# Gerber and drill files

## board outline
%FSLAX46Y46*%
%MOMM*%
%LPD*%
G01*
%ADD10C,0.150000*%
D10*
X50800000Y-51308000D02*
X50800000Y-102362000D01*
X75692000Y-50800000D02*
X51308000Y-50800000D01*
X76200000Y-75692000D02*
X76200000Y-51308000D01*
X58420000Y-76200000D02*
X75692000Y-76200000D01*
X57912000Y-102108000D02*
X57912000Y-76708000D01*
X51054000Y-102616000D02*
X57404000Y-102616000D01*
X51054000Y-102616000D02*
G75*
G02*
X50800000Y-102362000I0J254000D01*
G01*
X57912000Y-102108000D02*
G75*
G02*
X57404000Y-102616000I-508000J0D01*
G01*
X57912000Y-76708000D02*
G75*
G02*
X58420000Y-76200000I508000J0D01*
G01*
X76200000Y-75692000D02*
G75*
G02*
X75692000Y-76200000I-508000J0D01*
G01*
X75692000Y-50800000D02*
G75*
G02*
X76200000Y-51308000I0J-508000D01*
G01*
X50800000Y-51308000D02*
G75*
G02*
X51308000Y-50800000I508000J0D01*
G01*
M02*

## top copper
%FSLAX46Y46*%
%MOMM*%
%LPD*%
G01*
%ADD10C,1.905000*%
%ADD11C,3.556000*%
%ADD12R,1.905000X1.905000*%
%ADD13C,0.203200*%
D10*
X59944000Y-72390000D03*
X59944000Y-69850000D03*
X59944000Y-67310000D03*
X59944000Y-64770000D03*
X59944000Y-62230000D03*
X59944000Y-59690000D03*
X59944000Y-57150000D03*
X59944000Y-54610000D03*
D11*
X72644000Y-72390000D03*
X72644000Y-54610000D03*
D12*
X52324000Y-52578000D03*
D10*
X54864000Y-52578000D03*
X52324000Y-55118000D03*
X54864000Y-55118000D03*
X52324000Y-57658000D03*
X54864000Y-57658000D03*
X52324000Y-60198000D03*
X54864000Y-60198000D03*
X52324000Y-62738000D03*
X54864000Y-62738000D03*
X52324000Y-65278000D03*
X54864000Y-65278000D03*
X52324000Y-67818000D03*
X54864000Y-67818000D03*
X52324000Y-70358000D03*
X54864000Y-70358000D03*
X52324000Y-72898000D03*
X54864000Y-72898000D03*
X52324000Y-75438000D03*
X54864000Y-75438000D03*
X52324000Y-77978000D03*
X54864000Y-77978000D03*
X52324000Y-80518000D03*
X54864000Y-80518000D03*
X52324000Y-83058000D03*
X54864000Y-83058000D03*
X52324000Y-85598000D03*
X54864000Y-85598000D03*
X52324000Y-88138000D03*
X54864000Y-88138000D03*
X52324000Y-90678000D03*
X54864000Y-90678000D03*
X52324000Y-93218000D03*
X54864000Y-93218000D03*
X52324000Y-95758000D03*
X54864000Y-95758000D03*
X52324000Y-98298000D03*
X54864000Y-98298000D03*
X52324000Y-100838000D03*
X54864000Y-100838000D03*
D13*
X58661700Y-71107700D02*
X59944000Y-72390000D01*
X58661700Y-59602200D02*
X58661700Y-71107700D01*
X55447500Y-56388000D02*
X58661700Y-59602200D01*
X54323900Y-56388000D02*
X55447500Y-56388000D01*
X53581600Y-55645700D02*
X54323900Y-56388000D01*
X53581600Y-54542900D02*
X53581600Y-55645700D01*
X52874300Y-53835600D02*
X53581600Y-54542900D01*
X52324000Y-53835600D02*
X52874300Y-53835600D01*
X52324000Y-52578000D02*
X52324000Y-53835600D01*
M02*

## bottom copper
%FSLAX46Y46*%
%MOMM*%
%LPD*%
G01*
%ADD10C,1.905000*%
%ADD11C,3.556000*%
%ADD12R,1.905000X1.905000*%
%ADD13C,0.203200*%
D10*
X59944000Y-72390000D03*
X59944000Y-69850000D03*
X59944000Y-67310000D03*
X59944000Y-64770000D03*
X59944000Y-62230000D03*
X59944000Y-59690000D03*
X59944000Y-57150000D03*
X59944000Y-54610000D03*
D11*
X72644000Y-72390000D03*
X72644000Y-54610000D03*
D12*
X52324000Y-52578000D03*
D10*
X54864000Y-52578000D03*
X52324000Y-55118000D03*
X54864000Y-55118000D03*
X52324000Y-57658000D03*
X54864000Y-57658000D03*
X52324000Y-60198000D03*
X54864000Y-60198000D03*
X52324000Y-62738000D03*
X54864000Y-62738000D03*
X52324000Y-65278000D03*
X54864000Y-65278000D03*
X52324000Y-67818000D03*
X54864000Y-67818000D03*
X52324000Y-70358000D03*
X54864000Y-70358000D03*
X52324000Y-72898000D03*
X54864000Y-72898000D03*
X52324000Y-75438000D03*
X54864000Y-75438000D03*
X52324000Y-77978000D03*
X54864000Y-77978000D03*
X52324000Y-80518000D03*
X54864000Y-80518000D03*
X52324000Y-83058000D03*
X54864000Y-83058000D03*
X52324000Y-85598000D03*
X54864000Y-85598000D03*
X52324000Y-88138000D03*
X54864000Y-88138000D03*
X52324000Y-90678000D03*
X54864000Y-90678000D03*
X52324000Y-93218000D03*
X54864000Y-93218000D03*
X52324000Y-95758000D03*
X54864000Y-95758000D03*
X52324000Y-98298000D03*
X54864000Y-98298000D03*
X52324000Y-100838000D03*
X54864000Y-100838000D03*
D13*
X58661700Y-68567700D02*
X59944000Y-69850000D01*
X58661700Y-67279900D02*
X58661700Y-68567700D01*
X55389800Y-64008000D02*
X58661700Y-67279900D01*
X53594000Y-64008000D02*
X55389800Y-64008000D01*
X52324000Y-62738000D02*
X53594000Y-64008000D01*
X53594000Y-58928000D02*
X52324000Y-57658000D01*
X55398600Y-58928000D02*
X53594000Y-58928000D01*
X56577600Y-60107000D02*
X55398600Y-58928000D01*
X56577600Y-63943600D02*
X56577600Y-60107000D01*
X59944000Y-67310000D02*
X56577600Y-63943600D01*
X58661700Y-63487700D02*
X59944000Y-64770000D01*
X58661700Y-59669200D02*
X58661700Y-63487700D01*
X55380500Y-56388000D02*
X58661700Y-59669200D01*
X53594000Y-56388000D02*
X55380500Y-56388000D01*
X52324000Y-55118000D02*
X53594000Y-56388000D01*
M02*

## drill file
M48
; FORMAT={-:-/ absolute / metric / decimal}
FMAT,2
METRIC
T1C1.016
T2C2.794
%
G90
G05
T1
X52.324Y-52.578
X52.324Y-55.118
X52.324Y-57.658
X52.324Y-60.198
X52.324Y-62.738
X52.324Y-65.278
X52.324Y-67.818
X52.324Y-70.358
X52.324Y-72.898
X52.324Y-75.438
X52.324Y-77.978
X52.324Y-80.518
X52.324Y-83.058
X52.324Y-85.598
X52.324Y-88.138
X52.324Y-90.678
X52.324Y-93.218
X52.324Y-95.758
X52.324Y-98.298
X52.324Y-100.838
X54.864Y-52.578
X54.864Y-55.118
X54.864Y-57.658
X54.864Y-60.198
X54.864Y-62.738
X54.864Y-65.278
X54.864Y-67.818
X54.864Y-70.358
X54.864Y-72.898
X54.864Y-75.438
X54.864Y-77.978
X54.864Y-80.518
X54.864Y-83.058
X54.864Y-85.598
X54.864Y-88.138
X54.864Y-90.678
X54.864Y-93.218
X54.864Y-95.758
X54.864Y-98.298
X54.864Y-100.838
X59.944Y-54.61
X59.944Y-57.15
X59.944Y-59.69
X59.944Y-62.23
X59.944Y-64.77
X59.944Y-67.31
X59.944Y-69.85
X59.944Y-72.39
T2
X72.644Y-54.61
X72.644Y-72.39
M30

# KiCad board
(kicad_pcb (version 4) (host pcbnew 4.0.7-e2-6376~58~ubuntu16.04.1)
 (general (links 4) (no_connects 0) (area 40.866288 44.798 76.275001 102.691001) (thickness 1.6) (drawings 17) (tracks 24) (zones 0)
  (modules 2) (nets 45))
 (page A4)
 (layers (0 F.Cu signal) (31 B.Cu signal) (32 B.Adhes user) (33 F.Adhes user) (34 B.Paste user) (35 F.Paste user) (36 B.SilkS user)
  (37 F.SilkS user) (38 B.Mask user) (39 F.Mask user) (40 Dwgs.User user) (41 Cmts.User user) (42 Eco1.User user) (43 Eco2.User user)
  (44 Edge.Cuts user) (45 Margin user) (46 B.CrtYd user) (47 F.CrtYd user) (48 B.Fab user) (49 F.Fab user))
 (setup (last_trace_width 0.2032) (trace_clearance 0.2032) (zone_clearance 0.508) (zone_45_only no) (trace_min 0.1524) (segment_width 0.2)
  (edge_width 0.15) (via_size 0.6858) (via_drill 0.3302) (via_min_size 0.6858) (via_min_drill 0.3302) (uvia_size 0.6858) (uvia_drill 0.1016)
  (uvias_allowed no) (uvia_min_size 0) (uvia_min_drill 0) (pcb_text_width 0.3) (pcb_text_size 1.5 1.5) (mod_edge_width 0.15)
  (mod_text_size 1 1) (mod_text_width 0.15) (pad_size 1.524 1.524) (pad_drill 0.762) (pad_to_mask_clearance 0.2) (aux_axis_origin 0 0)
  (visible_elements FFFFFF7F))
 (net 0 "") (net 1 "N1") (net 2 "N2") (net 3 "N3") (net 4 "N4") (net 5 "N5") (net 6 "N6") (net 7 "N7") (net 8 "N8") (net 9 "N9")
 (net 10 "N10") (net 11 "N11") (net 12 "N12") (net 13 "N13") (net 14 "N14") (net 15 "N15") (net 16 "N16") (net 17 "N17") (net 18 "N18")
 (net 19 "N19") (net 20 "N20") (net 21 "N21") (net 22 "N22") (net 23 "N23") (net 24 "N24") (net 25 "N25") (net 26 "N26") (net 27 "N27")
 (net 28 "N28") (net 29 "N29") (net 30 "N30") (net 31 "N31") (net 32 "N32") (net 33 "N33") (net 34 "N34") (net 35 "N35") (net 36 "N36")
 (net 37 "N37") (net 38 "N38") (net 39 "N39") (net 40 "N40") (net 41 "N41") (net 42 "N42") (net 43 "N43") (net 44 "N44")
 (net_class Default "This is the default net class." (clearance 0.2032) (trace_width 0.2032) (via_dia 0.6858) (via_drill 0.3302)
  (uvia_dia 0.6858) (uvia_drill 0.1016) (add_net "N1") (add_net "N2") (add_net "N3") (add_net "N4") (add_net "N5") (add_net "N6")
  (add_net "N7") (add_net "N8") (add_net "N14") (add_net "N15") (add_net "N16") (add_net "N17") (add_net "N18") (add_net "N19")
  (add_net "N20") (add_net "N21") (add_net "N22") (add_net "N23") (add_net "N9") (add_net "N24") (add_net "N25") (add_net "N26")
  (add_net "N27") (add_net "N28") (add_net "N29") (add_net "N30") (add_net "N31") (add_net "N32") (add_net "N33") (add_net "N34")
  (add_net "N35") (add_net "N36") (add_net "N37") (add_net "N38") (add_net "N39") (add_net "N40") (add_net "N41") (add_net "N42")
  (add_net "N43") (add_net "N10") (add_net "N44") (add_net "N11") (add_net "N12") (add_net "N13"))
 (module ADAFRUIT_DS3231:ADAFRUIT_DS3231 (layer B.Cu) (at 59.944 63.5)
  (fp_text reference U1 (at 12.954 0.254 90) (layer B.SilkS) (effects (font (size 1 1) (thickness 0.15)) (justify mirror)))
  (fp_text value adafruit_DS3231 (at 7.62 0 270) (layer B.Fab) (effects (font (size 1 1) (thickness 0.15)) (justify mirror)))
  (pad 1 thru_hole circle (at 0 8.89) (size 1.905 1.905) (drill 1.016) (layers *.Cu *.Mask) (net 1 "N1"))
  (pad 2 thru_hole circle (at 0 6.35) (size 1.905 1.905) (drill 1.016) (layers *.Cu *.Mask) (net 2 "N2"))
  (pad 3 thru_hole circle (at 0 3.81) (size 1.905 1.905) (drill 1.016) (layers *.Cu *.Mask) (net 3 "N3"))
  (pad 4 thru_hole circle (at 0 1.27) (size 1.905 1.905) (drill 1.016) (layers *.Cu *.Mask) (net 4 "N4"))
  (pad 5 thru_hole circle (at 0 -1.27) (size 1.905 1.905) (drill 1.016) (layers *.Cu *.Mask) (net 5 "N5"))
  (pad 6 thru_hole circle (at 0 -3.81) (size 1.905 1.905) (drill 1.016) (layers *.Cu *.Mask) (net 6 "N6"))
  (pad 7 thru_hole circle (at 0 -6.35) (size 1.905 1.905) (drill 1.016) (layers *.Cu *.Mask) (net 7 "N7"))
  (pad 8 thru_hole circle (at 0 -8.89) (size 1.905 1.905) (drill 1.016) (layers *.Cu *.Mask) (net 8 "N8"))
  (pad "" thru_hole circle (at 12.7 8.89) (size 3.556 3.556) (drill 2.794) (layers *.Cu *.Mask))
  (pad "" thru_hole circle (at 12.7 -8.89) (size 3.556 3.556) (drill 2.794) (layers *.Cu *.Mask)))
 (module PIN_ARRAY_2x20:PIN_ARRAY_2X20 (layer F.Cu) (at 53.594 76.708)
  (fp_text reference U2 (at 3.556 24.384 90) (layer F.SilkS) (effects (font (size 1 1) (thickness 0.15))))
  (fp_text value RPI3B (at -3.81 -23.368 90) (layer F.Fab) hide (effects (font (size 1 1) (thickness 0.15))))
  (pad 1 thru_hole rect (at -1.27 -24.13) (size 1.905 1.905) (drill 1.016) (layers *.Cu *.Mask) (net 1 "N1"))
  (pad 2 thru_hole circle (at 1.27 -24.13) (size 1.905 1.905) (drill 1.016) (layers *.Cu *.Mask) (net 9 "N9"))
  (pad 3 thru_hole circle (at -1.27 -21.59) (size 1.905 1.905) (drill 1.016) (layers *.Cu *.Mask) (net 4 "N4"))
  (pad 4 thru_hole circle (at 1.27 -21.59) (size 1.905 1.905) (drill 1.016) (layers *.Cu *.Mask) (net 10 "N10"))
  (pad 5 thru_hole circle (at -1.27 -19.05) (size 1.905 1.905) (drill 1.016) (layers *.Cu *.Mask) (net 3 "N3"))
  (pad 6 thru_hole circle (at 1.27 -19.05) (size 1.905 1.905) (drill 1.016) (layers *.Cu *.Mask) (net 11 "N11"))
  (pad 7 thru_hole circle (at -1.27 -16.51) (size 1.905 1.905) (drill 1.016) (layers *.Cu *.Mask) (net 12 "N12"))
  (pad 8 thru_hole circle (at 1.27 -16.51) (size 1.905 1.905) (drill 1.016) (layers *.Cu *.Mask) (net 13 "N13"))
  (pad 9 thru_hole circle (at -1.27 -13.97) (size 1.905 1.905) (drill 1.016) (layers *.Cu *.Mask) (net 2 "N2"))
  (pad 10 thru_hole circle (at 1.27 -13.97) (size 1.905 1.905) (drill 1.016) (layers *.Cu *.Mask) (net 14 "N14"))
  (pad 11 thru_hole circle (at -1.27 -11.43) (size 1.905 1.905) (drill 1.016) (layers *.Cu *.Mask) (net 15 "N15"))
  (pad 12 thru_hole circle (at 1.27 -11.43) (size 1.905 1.905) (drill 1.016) (layers *.Cu *.Mask) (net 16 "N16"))
  (pad 13 thru_hole circle (at -1.27 -8.89) (size 1.905 1.905) (drill 1.016) (layers *.Cu *.Mask) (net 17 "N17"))
  (pad 14 thru_hole circle (at 1.27 -8.89) (size 1.905 1.905) (drill 1.016) (layers *.Cu *.Mask) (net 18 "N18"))
  (pad 15 thru_hole circle (at -1.27 -6.35) (size 1.905 1.905) (drill 1.016) (layers *.Cu *.Mask) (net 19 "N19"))
  (pad 16 thru_hole circle (at 1.27 -6.35) (size 1.905 1.905) (drill 1.016) (layers *.Cu *.Mask) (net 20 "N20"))
  (pad 17 thru_hole circle (at -1.27 -3.81) (size 1.905 1.905) (drill 1.016) (layers *.Cu *.Mask) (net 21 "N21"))
  (pad 18 thru_hole circle (at 1.27 -3.81) (size 1.905 1.905) (drill 1.016) (layers *.Cu *.Mask) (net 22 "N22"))
  (pad 19 thru_hole circle (at -1.27 -1.27) (size 1.905 1.905) (drill 1.016) (layers *.Cu *.Mask) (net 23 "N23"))
  (pad 20 thru_hole circle (at 1.27 -1.27) (size 1.905 1.905) (drill 1.016) (layers *.Cu *.Mask) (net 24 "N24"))
  (pad 21 thru_hole circle (at -1.27 1.27) (size 1.905 1.905) (drill 1.016) (layers *.Cu *.Mask) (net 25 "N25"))
  (pad 22 thru_hole circle (at 1.27 1.27) (size 1.905 1.905) (drill 1.016) (layers *.Cu *.Mask) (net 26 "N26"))
  (pad 23 thru_hole circle (at -1.27 3.81) (size 1.905 1.905) (drill 1.016) (layers *.Cu *.Mask) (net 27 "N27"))
  (pad 24 thru_hole circle (at 1.27 3.81) (size 1.905 1.905) (drill 1.016) (layers *.Cu *.Mask) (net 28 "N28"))
  (pad 25 thru_hole circle (at -1.27 6.35) (size 1.905 1.905) (drill 1.016) (layers *.Cu *.Mask) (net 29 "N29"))
  (pad 26 thru_hole circle (at 1.27 6.35) (size 1.905 1.905) (drill 1.016) (layers *.Cu *.Mask) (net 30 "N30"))
  (pad 27 thru_hole circle (at -1.27 8.89) (size 1.905 1.905) (drill 1.016) (layers *.Cu *.Mask) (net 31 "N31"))
  (pad 28 thru_hole circle (at 1.27 8.89) (size 1.905 1.905) (drill 1.016) (layers *.Cu *.Mask) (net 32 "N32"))
  (pad 29 thru_hole circle (at -1.27 11.43) (size 1.905 1.905) (drill 1.016) (layers *.Cu *.Mask) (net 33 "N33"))
  (pad 30 thru_hole circle (at 1.27 11.43) (size 1.905 1.905) (drill 1.016) (layers *.Cu *.Mask) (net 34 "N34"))
  (pad 31 thru_hole circle (at -1.27 13.97) (size 1.905 1.905) (drill 1.016) (layers *.Cu *.Mask) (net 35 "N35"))
  (pad 32 thru_hole circle (at 1.27 13.97) (size 1.905 1.905) (drill 1.016) (layers *.Cu *.Mask) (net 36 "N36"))
  (pad 33 thru_hole circle (at -1.27 16.51) (size 1.905 1.905) (drill 1.016) (layers *.Cu *.Mask) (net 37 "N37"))
  (pad 34 thru_hole circle (at 1.27 16.51) (size 1.905 1.905) (drill 1.016) (layers *.Cu *.Mask) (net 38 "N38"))
  (pad 35 thru_hole circle (at -1.27 19.05) (size 1.905 1.905) (drill 1.016) (layers *.Cu *.Mask) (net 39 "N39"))
  (pad 36 thru_hole circle (at 1.27 19.05) (size 1.905 1.905) (drill 1.016) (layers *.Cu *.Mask) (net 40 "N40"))
  (pad 37 thru_hole circle (at -1.27 21.59) (size 1.905 1.905) (drill 1.016) (layers *.Cu *.Mask) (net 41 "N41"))
  (pad 38 thru_hole circle (at 1.27 21.59) (size 1.905 1.905) (drill 1.016) (layers *.Cu *.Mask) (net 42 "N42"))
  (pad 39 thru_hole circle (at -1.27 24.13) (size 1.905 1.905) (drill 1.016) (layers *.Cu *.Mask) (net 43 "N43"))
  (pad 40 thru_hole circle (at 1.27 24.13) (size 1.905 1.905) (drill 1.016) (layers *.Cu *.Mask) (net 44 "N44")))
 (gr_line (start 50.8 51.308) (end 50.8 102.362) (angle 90) (layer Edge.Cuts) (width 0.15))
 (gr_line (start 75.692 50.8) (end 51.308 50.8) (angle 90) (layer Edge.Cuts) (width 0.15))
 (gr_line (start 76.2 75.692) (end 76.2 51.308) (angle 90) (layer Edge.Cuts) (width 0.15))
 (gr_line (start 58.42 76.2) (end 75.692 76.2) (angle 90) (layer Edge.Cuts) (width 0.15))
 (gr_line (start 57.912 102.108) (end 57.912 76.708) (angle 90) (layer Edge.Cuts) (width 0.15))
 (gr_line (start 51.054 102.616) (end 57.404 102.616) (angle 90) (layer Edge.Cuts) (width 0.15))
 (gr_arc (start 51.054 102.362) (end 51.054 102.616) (angle 90) (layer Edge.Cuts) (width 0.15))
 (gr_arc (start 57.404 102.108) (end 57.912 102.108) (angle 90) (layer Edge.Cuts) (width 0.15))
 (gr_arc (start 58.42 76.708) (end 57.912 76.708) (angle 90) (layer Edge.Cuts) (width 0.15))
 (gr_arc (start 75.692 75.692) (end 76.2 75.692) (angle 90) (layer Edge.Cuts) (width 0.15))
 (gr_arc (start 75.692 51.308) (end 75.692 50.8) (angle 90) (layer Edge.Cuts) (width 0.15))
 (gr_arc (start 51.308 51.308) (end 50.8 51.308) (angle 90) (layer Edge.Cuts) (width 0.15))
 (segment (start 58.6617 71.1077) (end 59.944 72.39) (width 0.2032) (layer F.Cu) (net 1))
 (segment (start 58.6617 59.6022) (end 58.6617 71.1077) (width 0.2032) (layer F.Cu) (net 1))
 (segment (start 55.4475 56.388) (end 58.6617 59.6022) (width 0.2032) (layer F.Cu) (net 1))
 (segment (start 54.3239 56.388) (end 55.4475 56.388) (width 0.2032) (layer F.Cu) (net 1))
 (segment (start 53.5816 55.6457) (end 54.3239 56.388) (width 0.2032) (layer F.Cu) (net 1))
 (segment (start 53.5816 54.5429) (end 53.5816 55.6457) (width 0.2032) (layer F.Cu) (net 1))
 (segment (start 52.8743 53.8356) (end 53.5816 54.5429) (width 0.2032) (layer F.Cu) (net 1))
 (segment (start 52.324 53.8356) (end 52.8743 53.8356) (width 0.2032) (layer F.Cu) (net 1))
 (segment (start 52.324 52.578) (end 52.324 53.8356) (width 0.2032) (layer F.Cu) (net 1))
 (segment (start 58.6617 68.5677) (end 59.944 69.85) (width 0.2032) (layer B.Cu) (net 2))
 (segment (start 58.6617 67.2799) (end 58.6617 68.5677) (width 0.2032) (layer B.Cu) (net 2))
 (segment (start 55.3898 64.008) (end 58.6617 67.2799) (width 0.2032) (layer B.Cu) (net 2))
 (segment (start 53.594 64.008) (end 55.3898 64.008) (width 0.2032) (layer B.Cu) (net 2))
 (segment (start 52.324 62.738) (end 53.594 64.008) (width 0.2032) (layer B.Cu) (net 2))
 (segment (start 53.594 58.928) (end 52.324 57.658) (width 0.2032) (layer B.Cu) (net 3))
 (segment (start 55.3986 58.928) (end 53.594 58.928) (width 0.2032) (layer B.Cu) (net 3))
 (segment (start 56.5776 60.107) (end 55.3986 58.928) (width 0.2032) (layer B.Cu) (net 3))
 (segment (start 56.5776 63.9436) (end 56.5776 60.107) (width 0.2032) (layer B.Cu) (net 3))
 (segment (start 59.944 67.31) (end 56.5776 63.9436) (width 0.2032) (layer B.Cu) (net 3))
 (segment (start 58.6617 63.4877) (end 59.944 64.77) (width 0.2032) (layer B.Cu) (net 4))
 (segment (start 58.6617 59.6692) (end 58.6617 63.4877) (width 0.2032) (layer B.Cu) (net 4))
 (segment (start 55.3805 56.388) (end 58.6617 59.6692) (width 0.2032) (layer B.Cu) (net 4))
 (segment (start 53.594 56.388) (end 55.3805 56.388) (width 0.2032) (layer B.Cu) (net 4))
 (segment (start 52.324 55.118) (end 53.594 56.388) (width 0.2032) (layer B.Cu) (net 4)))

